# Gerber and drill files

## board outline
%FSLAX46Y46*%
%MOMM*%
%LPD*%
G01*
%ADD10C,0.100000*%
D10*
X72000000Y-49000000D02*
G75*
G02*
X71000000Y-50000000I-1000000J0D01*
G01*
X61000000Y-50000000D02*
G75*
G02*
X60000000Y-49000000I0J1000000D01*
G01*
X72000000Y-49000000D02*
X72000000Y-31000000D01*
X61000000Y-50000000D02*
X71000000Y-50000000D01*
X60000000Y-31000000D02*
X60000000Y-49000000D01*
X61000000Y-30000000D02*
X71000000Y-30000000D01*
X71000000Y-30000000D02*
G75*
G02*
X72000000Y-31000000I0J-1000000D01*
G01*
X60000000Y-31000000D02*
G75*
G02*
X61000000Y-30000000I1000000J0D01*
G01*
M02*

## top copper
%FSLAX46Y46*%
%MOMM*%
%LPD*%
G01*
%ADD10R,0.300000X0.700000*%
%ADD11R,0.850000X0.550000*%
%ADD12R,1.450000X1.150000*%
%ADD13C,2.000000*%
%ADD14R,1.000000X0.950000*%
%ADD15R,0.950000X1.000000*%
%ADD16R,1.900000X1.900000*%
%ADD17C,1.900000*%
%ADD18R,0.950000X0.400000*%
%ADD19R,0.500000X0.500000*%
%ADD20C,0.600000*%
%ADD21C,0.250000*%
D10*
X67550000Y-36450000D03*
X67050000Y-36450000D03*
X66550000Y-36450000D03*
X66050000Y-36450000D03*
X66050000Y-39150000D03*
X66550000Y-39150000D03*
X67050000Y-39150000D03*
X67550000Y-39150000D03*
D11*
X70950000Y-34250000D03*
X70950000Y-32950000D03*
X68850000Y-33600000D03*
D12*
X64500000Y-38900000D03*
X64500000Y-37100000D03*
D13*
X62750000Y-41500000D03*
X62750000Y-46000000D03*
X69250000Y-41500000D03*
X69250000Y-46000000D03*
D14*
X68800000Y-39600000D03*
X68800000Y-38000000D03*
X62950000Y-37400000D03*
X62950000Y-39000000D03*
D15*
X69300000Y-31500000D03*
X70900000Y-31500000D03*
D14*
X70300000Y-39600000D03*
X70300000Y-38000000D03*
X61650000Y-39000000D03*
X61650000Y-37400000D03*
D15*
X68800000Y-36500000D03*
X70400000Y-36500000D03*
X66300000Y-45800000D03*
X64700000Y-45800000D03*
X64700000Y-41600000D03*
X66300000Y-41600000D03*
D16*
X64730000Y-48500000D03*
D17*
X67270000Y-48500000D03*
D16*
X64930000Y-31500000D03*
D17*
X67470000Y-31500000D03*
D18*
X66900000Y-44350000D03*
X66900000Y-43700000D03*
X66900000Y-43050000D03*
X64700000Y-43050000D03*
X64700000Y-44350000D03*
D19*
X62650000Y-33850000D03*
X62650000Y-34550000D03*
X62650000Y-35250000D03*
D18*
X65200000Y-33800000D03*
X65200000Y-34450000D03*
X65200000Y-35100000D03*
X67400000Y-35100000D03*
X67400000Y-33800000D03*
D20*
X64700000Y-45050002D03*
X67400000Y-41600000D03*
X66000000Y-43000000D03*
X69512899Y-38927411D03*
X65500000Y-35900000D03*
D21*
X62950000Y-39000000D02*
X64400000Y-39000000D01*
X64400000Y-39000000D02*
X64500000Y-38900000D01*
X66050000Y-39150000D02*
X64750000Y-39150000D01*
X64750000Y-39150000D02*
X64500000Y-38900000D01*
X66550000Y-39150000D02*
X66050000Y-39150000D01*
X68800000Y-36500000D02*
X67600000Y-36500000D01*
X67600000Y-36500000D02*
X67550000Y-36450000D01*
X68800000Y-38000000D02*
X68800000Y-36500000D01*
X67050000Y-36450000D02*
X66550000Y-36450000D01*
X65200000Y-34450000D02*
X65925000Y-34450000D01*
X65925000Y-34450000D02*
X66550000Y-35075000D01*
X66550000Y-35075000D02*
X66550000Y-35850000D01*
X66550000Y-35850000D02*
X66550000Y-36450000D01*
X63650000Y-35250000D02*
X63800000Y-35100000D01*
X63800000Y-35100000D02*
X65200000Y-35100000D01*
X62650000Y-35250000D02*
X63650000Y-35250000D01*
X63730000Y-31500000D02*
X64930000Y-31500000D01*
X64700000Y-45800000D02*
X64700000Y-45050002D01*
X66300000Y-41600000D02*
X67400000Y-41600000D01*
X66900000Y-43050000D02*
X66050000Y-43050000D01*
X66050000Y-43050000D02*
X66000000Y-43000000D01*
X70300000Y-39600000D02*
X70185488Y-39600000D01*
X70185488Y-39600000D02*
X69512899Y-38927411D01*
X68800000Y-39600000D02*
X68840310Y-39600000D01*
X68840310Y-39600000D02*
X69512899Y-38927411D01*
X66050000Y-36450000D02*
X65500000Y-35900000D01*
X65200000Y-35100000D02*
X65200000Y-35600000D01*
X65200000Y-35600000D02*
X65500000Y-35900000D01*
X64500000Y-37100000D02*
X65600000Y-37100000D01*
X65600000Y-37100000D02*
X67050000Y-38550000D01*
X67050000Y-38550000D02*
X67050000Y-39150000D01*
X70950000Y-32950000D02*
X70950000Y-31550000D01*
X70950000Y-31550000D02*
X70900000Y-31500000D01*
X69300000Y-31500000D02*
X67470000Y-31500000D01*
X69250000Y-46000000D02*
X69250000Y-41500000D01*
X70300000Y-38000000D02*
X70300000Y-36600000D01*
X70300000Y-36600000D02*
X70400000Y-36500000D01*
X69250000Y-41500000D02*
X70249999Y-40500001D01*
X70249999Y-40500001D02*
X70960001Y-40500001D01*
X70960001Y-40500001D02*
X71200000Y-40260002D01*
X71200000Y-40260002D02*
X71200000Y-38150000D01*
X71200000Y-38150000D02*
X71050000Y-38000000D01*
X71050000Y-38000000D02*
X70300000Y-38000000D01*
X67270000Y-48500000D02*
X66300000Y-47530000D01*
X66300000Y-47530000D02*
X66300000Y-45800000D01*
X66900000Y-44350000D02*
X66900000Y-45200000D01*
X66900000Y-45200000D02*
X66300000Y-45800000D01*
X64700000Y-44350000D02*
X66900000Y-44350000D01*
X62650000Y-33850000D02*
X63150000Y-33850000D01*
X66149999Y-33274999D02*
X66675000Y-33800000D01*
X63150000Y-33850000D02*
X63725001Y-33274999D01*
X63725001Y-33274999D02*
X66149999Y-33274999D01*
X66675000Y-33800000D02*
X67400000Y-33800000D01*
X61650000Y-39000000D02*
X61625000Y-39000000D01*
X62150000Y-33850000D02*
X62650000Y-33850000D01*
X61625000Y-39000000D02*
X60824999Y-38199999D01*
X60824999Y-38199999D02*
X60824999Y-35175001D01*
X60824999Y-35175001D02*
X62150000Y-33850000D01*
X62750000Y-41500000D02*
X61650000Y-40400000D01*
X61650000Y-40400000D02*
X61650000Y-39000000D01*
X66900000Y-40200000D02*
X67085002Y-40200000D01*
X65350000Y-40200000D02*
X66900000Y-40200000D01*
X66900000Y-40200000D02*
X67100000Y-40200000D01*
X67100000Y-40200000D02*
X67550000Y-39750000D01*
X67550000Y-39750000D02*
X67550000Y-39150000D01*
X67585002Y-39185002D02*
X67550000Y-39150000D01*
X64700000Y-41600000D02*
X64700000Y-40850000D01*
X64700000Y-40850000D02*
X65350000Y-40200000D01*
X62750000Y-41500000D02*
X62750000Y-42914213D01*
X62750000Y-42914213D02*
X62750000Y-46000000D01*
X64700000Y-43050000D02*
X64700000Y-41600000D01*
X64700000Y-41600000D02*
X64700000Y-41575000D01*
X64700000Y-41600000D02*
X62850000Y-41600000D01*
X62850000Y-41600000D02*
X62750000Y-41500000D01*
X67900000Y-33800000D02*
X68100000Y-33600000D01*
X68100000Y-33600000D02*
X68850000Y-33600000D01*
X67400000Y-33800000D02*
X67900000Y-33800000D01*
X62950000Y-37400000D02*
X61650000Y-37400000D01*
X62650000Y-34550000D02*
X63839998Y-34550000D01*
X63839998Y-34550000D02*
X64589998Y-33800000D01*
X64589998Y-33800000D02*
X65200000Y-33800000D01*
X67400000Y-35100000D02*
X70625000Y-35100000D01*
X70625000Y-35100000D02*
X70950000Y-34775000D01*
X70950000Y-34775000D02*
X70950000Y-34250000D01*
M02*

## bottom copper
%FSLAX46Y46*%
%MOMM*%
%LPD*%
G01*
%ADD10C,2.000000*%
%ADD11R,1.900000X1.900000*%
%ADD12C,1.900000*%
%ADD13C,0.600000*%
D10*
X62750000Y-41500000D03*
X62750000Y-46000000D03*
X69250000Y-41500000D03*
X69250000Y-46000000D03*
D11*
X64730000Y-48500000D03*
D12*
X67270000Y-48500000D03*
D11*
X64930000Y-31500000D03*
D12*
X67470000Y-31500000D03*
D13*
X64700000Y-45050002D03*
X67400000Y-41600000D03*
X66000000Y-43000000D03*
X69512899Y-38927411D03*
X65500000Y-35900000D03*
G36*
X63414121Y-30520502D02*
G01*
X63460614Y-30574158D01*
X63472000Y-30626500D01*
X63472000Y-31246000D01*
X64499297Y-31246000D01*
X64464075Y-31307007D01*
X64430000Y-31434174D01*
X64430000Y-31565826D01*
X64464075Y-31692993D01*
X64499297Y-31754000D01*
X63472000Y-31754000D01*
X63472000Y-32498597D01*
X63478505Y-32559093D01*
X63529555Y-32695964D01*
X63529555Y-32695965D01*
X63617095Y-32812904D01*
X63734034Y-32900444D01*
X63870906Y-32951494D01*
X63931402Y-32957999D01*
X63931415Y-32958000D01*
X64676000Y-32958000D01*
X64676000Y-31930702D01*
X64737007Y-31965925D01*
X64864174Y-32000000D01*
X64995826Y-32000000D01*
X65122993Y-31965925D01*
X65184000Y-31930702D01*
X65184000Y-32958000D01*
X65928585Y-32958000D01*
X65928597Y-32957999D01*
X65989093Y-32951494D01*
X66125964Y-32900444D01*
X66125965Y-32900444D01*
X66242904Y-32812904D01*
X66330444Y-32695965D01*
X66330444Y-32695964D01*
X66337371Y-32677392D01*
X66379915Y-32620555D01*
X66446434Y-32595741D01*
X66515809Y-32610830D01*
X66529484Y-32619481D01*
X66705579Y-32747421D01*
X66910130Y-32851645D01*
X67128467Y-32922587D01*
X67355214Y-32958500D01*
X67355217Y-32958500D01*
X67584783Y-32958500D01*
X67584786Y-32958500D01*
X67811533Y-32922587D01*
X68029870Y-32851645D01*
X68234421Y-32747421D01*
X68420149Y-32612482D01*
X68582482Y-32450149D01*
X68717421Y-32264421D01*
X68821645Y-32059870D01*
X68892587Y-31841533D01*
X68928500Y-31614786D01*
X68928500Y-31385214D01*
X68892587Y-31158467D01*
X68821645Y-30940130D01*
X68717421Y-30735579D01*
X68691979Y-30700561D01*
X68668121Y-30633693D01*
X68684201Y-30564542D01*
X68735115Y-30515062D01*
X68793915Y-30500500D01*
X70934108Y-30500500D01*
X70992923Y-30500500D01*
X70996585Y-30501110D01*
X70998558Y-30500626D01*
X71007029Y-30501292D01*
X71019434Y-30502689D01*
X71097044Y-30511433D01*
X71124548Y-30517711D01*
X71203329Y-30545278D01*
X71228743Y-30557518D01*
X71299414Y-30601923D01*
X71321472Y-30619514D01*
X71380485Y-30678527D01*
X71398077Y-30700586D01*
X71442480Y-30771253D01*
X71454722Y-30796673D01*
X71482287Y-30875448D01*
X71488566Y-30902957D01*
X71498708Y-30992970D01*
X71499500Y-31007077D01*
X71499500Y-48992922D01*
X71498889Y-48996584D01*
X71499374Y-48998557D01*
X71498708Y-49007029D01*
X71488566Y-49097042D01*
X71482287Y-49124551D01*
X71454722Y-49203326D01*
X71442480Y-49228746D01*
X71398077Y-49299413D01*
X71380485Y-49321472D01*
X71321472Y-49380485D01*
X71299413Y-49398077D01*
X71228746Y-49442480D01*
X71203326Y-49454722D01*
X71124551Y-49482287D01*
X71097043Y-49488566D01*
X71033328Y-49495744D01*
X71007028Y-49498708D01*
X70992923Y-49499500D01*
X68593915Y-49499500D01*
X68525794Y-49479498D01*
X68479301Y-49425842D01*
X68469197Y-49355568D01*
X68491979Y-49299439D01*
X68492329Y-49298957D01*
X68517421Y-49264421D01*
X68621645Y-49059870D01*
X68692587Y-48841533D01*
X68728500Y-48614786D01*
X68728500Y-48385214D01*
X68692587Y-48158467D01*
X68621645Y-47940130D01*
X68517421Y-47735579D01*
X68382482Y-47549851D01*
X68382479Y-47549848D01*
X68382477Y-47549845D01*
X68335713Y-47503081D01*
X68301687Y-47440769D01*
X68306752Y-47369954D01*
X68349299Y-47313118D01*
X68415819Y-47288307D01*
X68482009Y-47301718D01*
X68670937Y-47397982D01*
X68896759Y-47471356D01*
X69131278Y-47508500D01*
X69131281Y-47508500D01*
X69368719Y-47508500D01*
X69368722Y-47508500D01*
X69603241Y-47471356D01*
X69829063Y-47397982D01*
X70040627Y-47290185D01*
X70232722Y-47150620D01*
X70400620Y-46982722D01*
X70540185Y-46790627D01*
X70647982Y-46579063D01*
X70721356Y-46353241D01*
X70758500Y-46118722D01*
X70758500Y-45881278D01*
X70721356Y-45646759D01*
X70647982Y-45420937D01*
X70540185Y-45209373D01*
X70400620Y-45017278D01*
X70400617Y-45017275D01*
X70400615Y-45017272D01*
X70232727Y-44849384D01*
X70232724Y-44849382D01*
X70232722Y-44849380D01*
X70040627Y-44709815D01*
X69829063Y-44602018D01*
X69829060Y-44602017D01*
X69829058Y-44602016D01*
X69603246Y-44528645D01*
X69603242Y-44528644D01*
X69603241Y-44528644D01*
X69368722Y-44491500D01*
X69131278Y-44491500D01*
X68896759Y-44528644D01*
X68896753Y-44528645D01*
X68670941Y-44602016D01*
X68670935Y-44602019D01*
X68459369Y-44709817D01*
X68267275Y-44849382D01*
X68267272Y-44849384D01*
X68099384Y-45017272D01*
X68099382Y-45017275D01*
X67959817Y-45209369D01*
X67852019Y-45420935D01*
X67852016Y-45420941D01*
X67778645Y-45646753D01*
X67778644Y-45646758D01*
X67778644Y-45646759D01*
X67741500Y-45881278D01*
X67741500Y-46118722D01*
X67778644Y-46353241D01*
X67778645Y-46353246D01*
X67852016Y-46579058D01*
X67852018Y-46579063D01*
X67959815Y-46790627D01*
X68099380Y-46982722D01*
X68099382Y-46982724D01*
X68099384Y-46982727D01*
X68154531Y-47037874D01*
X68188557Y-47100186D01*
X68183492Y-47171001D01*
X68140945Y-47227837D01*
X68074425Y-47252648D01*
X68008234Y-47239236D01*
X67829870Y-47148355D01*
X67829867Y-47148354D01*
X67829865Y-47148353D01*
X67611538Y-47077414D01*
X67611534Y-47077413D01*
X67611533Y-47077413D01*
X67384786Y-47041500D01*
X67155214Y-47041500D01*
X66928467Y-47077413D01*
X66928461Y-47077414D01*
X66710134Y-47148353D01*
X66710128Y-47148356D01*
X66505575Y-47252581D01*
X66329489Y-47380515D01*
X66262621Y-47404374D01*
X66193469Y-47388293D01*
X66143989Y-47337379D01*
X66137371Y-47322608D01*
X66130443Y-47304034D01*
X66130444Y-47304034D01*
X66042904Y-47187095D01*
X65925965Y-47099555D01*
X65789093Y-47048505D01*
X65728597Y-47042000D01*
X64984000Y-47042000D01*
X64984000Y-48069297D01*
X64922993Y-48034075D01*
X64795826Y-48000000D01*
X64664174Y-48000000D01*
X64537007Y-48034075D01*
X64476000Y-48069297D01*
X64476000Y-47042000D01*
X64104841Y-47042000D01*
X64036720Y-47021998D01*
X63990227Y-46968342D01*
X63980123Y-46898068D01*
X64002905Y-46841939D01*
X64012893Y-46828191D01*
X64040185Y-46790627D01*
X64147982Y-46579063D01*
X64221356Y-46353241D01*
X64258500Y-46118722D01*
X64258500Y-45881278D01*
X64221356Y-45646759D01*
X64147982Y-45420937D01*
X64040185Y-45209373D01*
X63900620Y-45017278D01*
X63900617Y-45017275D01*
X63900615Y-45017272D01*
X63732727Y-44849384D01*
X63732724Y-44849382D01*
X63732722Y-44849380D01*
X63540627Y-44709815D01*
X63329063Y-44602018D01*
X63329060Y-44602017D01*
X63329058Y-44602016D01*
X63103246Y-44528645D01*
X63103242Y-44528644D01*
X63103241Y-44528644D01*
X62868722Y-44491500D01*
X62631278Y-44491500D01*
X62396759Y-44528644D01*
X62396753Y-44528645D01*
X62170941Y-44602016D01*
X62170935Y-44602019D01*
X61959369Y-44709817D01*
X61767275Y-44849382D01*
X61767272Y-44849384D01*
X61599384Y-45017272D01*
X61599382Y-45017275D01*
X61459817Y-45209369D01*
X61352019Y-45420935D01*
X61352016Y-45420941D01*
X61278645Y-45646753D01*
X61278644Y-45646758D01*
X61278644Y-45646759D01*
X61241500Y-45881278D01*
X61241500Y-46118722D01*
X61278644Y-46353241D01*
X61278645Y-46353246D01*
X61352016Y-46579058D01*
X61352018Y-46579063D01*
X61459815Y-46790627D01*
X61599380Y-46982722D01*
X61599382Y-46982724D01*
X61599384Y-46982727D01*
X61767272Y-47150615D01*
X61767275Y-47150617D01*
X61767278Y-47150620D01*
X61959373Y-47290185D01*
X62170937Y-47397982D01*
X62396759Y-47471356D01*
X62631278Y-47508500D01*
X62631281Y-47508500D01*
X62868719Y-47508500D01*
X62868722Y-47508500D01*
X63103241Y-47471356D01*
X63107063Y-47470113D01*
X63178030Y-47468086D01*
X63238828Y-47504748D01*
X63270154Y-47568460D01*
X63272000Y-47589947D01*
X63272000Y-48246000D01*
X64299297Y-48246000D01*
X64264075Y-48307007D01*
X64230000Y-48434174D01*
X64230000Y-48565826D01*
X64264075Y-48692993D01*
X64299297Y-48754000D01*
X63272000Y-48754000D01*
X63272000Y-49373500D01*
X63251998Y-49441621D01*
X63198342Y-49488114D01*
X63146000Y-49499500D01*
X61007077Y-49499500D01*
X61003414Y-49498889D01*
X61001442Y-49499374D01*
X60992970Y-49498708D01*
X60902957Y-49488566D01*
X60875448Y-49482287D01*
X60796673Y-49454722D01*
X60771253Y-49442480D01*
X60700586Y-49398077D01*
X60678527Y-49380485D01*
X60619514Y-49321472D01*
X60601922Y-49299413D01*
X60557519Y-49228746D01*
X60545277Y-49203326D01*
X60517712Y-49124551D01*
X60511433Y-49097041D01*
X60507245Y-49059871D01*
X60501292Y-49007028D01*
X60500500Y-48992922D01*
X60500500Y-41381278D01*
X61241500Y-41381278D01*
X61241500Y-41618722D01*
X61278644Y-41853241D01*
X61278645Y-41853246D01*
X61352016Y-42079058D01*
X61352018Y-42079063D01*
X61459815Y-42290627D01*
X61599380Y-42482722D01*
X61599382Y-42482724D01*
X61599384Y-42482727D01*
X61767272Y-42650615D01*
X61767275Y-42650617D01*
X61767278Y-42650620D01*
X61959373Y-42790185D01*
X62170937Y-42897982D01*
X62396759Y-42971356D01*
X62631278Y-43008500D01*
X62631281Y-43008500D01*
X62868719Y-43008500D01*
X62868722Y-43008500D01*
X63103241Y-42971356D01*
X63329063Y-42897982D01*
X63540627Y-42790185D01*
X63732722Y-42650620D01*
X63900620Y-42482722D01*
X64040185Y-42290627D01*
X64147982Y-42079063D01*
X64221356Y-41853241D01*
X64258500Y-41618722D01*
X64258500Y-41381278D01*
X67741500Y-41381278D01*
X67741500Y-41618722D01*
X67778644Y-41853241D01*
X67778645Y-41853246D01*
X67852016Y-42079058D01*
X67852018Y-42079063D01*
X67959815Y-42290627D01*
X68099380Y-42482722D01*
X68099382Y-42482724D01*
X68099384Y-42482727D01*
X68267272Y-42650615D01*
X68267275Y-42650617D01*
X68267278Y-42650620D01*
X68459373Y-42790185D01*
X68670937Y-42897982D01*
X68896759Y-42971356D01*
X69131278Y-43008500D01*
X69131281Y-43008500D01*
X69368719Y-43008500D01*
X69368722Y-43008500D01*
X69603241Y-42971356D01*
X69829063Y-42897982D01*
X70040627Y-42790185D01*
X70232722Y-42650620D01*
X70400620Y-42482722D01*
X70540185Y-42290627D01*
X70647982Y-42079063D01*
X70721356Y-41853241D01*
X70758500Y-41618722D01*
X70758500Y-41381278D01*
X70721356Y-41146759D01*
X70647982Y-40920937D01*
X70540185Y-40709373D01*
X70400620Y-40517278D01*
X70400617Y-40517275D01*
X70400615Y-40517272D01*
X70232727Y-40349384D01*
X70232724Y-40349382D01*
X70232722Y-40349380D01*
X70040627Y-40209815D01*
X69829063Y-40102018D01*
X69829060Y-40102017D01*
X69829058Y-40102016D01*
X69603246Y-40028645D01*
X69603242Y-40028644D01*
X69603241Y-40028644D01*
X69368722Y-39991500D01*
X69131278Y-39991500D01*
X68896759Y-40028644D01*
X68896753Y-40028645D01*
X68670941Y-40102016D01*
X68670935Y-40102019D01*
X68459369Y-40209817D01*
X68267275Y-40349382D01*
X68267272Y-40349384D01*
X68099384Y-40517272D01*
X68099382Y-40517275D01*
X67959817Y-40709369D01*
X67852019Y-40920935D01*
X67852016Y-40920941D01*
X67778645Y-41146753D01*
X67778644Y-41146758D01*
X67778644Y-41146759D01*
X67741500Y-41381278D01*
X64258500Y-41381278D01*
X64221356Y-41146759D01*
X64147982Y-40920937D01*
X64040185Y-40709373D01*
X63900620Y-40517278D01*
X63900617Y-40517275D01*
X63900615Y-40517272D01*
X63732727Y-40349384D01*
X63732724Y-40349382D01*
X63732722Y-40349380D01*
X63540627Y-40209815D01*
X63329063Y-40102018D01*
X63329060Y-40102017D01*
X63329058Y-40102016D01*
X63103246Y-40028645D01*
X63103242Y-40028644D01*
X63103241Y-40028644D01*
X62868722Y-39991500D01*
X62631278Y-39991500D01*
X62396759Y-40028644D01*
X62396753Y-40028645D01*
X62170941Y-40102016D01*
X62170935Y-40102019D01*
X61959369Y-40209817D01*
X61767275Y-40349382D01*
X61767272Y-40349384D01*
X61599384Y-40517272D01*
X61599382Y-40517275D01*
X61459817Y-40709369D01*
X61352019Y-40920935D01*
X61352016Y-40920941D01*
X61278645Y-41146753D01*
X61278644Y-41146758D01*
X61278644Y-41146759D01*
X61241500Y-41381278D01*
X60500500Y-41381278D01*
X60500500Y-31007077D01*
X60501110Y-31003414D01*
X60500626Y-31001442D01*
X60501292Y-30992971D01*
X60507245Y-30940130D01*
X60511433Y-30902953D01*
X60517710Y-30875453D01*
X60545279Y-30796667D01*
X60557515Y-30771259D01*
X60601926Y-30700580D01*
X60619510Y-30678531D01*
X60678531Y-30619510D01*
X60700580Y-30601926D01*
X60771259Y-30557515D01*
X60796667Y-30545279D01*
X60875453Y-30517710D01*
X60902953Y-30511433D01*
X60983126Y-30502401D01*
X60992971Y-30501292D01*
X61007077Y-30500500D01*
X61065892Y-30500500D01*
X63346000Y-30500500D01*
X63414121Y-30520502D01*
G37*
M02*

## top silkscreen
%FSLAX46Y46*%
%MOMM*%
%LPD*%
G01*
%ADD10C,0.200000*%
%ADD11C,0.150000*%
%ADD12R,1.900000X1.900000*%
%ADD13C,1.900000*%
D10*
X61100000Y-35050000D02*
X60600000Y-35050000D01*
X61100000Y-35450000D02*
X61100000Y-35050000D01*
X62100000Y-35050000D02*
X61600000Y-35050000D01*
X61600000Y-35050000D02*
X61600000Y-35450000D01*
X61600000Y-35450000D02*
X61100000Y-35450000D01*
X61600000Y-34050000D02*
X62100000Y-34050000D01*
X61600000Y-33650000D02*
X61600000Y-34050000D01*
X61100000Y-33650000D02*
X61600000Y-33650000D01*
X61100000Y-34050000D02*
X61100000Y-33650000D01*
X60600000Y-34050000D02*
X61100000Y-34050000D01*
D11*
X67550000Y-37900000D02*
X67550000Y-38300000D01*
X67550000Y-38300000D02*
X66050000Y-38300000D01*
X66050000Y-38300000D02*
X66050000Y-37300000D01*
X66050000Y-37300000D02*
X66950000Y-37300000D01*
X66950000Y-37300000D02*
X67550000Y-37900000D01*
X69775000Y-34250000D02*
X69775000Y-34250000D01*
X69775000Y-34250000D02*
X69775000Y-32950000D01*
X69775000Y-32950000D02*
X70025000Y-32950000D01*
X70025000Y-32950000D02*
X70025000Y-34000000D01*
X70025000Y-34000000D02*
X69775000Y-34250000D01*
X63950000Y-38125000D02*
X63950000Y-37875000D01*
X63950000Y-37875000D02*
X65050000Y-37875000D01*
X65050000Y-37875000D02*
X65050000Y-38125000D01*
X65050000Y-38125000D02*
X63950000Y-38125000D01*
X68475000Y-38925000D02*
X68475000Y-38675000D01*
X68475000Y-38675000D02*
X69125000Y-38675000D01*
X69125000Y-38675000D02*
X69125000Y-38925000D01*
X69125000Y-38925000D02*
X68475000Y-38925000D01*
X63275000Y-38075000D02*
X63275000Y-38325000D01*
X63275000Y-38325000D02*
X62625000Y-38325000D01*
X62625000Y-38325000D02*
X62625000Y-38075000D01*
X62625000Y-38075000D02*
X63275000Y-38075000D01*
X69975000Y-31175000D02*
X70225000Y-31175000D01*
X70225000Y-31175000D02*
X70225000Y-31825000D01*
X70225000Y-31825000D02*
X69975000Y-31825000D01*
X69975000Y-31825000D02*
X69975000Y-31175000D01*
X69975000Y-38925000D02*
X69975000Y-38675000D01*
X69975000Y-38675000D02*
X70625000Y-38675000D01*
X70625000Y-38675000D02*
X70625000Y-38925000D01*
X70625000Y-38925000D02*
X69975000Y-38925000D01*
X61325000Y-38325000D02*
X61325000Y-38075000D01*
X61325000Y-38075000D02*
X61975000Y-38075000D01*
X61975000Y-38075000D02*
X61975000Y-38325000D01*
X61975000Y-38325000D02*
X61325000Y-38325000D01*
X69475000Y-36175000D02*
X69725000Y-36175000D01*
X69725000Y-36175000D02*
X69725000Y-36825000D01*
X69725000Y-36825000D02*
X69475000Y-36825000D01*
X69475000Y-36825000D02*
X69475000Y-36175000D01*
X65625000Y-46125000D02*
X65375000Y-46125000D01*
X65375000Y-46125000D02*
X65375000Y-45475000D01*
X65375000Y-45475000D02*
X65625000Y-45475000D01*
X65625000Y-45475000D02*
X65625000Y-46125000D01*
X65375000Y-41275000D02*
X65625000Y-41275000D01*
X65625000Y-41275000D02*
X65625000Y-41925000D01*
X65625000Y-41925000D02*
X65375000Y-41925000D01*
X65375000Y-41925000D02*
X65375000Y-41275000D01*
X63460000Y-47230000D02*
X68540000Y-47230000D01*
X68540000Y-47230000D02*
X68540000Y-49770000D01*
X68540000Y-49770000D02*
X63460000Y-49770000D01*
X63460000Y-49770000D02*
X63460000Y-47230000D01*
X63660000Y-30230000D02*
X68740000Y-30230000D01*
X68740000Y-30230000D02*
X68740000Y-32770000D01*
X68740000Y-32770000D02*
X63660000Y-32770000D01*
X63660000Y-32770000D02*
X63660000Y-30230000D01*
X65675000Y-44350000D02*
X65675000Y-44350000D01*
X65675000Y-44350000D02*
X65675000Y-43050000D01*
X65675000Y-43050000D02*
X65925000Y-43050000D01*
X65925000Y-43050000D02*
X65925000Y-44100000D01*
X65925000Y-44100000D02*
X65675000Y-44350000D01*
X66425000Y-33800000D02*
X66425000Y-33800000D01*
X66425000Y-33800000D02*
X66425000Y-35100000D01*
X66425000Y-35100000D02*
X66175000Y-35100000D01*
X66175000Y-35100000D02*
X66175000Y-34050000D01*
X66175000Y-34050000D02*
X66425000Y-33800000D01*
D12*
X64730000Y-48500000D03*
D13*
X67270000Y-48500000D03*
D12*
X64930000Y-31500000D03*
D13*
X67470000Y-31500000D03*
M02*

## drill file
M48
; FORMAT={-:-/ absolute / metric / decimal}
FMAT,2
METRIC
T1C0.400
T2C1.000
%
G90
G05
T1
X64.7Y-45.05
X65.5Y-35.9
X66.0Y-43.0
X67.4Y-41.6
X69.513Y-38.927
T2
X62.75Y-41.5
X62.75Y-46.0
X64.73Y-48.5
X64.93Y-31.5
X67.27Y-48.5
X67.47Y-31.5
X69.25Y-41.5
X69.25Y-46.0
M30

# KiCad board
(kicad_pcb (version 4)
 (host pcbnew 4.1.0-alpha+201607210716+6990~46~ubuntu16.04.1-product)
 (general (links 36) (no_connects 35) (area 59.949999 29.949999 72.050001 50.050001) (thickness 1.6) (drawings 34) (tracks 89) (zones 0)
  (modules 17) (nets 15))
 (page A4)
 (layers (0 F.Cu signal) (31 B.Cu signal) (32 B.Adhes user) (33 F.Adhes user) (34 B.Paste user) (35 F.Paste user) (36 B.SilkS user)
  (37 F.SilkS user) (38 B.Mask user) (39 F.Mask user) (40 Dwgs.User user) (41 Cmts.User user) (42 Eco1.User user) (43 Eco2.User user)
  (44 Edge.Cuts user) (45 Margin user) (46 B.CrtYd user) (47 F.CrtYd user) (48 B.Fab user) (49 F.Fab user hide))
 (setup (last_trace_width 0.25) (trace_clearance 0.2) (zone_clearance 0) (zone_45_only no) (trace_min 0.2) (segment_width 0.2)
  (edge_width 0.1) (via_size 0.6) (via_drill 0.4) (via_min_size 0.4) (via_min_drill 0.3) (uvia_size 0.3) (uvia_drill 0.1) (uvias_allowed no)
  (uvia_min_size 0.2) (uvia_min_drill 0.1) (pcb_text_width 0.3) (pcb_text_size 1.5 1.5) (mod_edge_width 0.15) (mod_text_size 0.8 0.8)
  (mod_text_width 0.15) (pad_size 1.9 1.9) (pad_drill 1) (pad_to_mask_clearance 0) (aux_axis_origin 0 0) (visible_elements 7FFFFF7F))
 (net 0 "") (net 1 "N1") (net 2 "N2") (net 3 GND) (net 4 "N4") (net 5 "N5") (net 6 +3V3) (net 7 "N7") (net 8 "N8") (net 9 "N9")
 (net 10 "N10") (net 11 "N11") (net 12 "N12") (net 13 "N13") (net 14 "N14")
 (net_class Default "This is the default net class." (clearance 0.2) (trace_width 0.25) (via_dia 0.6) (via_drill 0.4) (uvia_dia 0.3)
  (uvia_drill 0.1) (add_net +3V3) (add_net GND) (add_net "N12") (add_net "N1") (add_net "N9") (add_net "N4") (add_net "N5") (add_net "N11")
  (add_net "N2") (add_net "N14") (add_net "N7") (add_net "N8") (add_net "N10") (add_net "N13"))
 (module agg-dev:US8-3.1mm (layer F.Cu) (at 66.8 37.8 270)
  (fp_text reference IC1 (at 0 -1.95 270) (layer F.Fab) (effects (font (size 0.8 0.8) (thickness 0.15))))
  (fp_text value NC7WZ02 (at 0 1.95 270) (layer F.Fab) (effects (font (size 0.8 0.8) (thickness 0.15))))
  (fp_line (start 0.1 -0.75) (end 0.5 -0.75) (layer F.SilkS) (width 0.15))
  (fp_line (start 0.5 -0.75) (end 0.5 0.75) (layer F.SilkS) (width 0.15))
  (fp_line (start 0.5 0.75) (end -0.5 0.75) (layer F.SilkS) (width 0.15))
  (fp_line (start -0.5 0.75) (end -0.5 -0.15) (layer F.SilkS) (width 0.15))
  (fp_line (start -0.5 -0.15) (end 0.1 -0.75) (layer F.SilkS) (width 0.15))
  (pad 1 smd rect (at -1.35 -0.75 270) (size 0.7 0.3) (layers F.Cu F.Paste F.Mask) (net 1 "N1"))
  (pad 2 smd rect (at -1.35 -0.25 270) (size 0.7 0.3) (layers F.Cu F.Paste F.Mask) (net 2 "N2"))
  (pad 3 smd rect (at -1.35 0.25 270) (size 0.7 0.3) (layers F.Cu F.Paste F.Mask) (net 2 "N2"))
  (pad 4 smd rect (at -1.35 0.75 270) (size 0.7 0.3) (layers F.Cu F.Paste F.Mask) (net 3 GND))
  (pad 5 smd rect (at 1.35 0.75 270) (size 0.7 0.3) (layers F.Cu F.Paste F.Mask) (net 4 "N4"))
  (pad 6 smd rect (at 1.35 0.25 270) (size 0.7 0.3) (layers F.Cu F.Paste F.Mask) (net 4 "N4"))
  (pad 7 smd rect (at 1.35 -0.25 270) (size 0.7 0.3) (layers F.Cu F.Paste F.Mask) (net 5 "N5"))
  (pad 8 smd rect (at 1.35 -0.75 270) (size 0.7 0.3) (layers F.Cu F.Paste F.Mask) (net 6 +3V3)))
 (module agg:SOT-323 (layer F.Cu) (at 69.9 33.6 180)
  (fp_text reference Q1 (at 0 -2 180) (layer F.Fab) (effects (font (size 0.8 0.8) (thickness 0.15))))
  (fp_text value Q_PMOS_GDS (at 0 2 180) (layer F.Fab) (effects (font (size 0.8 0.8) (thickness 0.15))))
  (fp_line (start 0.125 -0.65) (end 0.125 -0.65) (layer F.SilkS) (width 0.15))
  (fp_line (start 0.125 -0.65) (end 0.125 0.65) (layer F.SilkS) (width 0.15))
  (fp_line (start 0.125 0.65) (end -0.125 0.65) (layer F.SilkS) (width 0.15))
  (fp_line (start -0.125 0.65) (end -0.125 -0.4) (layer F.SilkS) (width 0.15))
  (fp_line (start -0.125 -0.4) (end 0.125 -0.65) (layer F.SilkS) (width 0.15))
  (pad 1 smd rect (at -1.05 -0.65 180) (size 0.85 0.55) (layers F.Cu F.Paste F.Mask) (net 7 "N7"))
  (pad 2 smd rect (at -1.05 0.65 180) (size 0.85 0.55) (layers F.Cu F.Paste F.Mask) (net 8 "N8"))
  (pad 3 smd rect (at 1.05 0 180) (size 0.85 0.55) (layers F.Cu F.Paste F.Mask) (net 6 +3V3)))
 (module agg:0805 (layer F.Cu) (at 64.5 38 90)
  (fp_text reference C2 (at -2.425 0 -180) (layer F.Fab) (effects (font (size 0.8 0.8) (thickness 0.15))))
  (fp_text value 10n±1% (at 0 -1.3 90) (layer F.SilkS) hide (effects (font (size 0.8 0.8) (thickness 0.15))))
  (fp_line (start -0.125 -0.55) (end 0.125 -0.55) (layer F.SilkS) (width 0.15))
  (fp_line (start 0.125 -0.55) (end 0.125 0.55) (layer F.SilkS) (width 0.15))
  (fp_line (start 0.125 0.55) (end -0.125 0.55) (layer F.SilkS) (width 0.15))
  (fp_line (start -0.125 0.55) (end -0.125 -0.55) (layer F.SilkS) (width 0.15))
  (pad 1 smd rect (at -0.9 0 90) (size 1.15 1.45) (layers F.Cu F.Paste F.Mask) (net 4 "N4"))
  (pad 2 smd rect (at 0.9 0 90) (size 1.15 1.45) (layers F.Cu F.Paste F.Mask) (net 5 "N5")))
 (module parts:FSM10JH (layer B.Cu) (at 62.75 41.5 180)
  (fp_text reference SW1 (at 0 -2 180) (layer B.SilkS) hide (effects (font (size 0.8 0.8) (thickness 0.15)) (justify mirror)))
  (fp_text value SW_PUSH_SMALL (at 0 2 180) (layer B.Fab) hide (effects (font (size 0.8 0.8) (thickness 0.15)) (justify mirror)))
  (pad 1 thru_hole circle (at 0 0 180) (size 2 2) (drill 1) (layers *.Cu *.Mask B.SilkS) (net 6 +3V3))
  (pad 1 thru_hole circle (at 0 -4.5 180) (size 2 2) (drill 1) (layers *.Cu *.Mask B.SilkS) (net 6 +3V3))
  (pad 2 thru_hole circle (at -6.5 0 180) (size 2 2) (drill 1) (layers *.Cu *.Mask B.SilkS) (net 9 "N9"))
  (pad 2 thru_hole circle (at -6.5 -4.5 180) (size 2 2) (drill 1) (layers *.Cu *.Mask B.SilkS) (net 9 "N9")))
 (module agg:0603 (layer F.Cu) (at 68.8 38.8 90)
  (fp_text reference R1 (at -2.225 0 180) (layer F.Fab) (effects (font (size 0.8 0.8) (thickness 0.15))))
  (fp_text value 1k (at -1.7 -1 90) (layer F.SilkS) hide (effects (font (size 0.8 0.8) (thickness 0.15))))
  (fp_line (start -0.125 -0.325) (end 0.125 -0.325) (layer F.SilkS) (width 0.15))
  (fp_line (start 0.125 -0.325) (end 0.125 0.325) (layer F.SilkS) (width 0.15))
  (fp_line (start 0.125 0.325) (end -0.125 0.325) (layer F.SilkS) (width 0.15))
  (fp_line (start -0.125 0.325) (end -0.125 -0.325) (layer F.SilkS) (width 0.15))
  (pad 1 smd rect (at -0.8 0 90) (size 0.95 1) (layers F.Cu F.Paste F.Mask) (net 3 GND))
  (pad 2 smd rect (at 0.8 0 90) (size 0.95 1) (layers F.Cu F.Paste F.Mask) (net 1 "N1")))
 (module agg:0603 (layer F.Cu) (at 62.95 38.2 270)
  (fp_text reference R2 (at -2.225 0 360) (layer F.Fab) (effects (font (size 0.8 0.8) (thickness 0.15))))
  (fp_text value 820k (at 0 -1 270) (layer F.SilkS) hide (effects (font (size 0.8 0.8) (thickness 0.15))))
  (fp_line (start -0.125 -0.325) (end 0.125 -0.325) (layer F.SilkS) (width 0.15))
  (fp_line (start 0.125 -0.325) (end 0.125 0.325) (layer F.SilkS) (width 0.15))
  (fp_line (start 0.125 0.325) (end -0.125 0.325) (layer F.SilkS) (width 0.15))
  (fp_line (start -0.125 0.325) (end -0.125 -0.325) (layer F.SilkS) (width 0.15))
  (pad 1 smd rect (at -0.8 0 270) (size 0.95 1) (layers F.Cu F.Paste F.Mask) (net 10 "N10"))
  (pad 2 smd rect (at 0.8 0 270) (size 0.95 1) (layers F.Cu F.Paste F.Mask) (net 4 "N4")))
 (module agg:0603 (layer F.Cu) (at 70.1 31.5)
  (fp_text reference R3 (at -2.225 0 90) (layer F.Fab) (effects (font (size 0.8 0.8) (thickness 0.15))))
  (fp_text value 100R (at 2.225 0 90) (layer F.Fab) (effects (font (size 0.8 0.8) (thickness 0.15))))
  (fp_line (start -0.125 -0.325) (end 0.125 -0.325) (layer F.SilkS) (width 0.15))
  (fp_line (start 0.125 -0.325) (end 0.125 0.325) (layer F.SilkS) (width 0.15))
  (fp_line (start 0.125 0.325) (end -0.125 0.325) (layer F.SilkS) (width 0.15))
  (fp_line (start -0.125 0.325) (end -0.125 -0.325) (layer F.SilkS) (width 0.15))
  (pad 1 smd rect (at -0.8 0) (size 0.95 1) (layers F.Cu F.Paste F.Mask) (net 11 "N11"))
  (pad 2 smd rect (at 0.8 0) (size 0.95 1) (layers F.Cu F.Paste F.Mask) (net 8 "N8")))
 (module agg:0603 (layer F.Cu) (at 70.3 38.8 90)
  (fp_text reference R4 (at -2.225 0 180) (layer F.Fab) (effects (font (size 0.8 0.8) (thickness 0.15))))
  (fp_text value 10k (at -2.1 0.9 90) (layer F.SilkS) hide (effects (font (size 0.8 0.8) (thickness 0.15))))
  (fp_line (start -0.125 -0.325) (end 0.125 -0.325) (layer F.SilkS) (width 0.15))
  (fp_line (start 0.125 -0.325) (end 0.125 0.325) (layer F.SilkS) (width 0.15))
  (fp_line (start 0.125 0.325) (end -0.125 0.325) (layer F.SilkS) (width 0.15))
  (fp_line (start -0.125 0.325) (end -0.125 -0.325) (layer F.SilkS) (width 0.15))
  (pad 1 smd rect (at -0.8 0 90) (size 0.95 1) (layers F.Cu F.Paste F.Mask) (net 3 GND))
  (pad 2 smd rect (at 0.8 0 90) (size 0.95 1) (layers F.Cu F.Paste F.Mask) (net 9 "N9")))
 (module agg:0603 (layer F.Cu) (at 61.65 38.2 90)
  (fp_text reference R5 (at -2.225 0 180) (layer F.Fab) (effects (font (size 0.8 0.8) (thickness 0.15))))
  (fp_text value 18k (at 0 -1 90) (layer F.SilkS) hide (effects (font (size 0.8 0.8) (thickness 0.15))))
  (fp_line (start -0.125 -0.325) (end 0.125 -0.325) (layer F.SilkS) (width 0.15))
  (fp_line (start 0.125 -0.325) (end 0.125 0.325) (layer F.SilkS) (width 0.15))
  (fp_line (start 0.125 0.325) (end -0.125 0.325) (layer F.SilkS) (width 0.15))
  (fp_line (start -0.125 0.325) (end -0.125 -0.325) (layer F.SilkS) (width 0.15))
  (pad 1 smd rect (at -0.8 0 90) (size 0.95 1) (layers F.Cu F.Paste F.Mask) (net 6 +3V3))
  (pad 2 smd rect (at 0.8 0 90) (size 0.95 1) (layers F.Cu F.Paste F.Mask) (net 10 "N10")))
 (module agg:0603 (layer F.Cu) (at 69.6 36.5)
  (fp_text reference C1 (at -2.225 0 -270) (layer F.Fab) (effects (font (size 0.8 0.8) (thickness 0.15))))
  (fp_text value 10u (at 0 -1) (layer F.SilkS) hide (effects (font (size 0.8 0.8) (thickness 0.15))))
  (fp_line (start -0.125 -0.325) (end 0.125 -0.325) (layer F.SilkS) (width 0.15))
  (fp_line (start 0.125 -0.325) (end 0.125 0.325) (layer F.SilkS) (width 0.15))
  (fp_line (start 0.125 0.325) (end -0.125 0.325) (layer F.SilkS) (width 0.15))
  (fp_line (start -0.125 0.325) (end -0.125 -0.325) (layer F.SilkS) (width 0.15))
  (pad 1 smd rect (at -0.8 0) (size 0.95 1) (layers F.Cu F.Paste F.Mask) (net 1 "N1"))
  (pad 2 smd rect (at 0.8 0) (size 0.95 1) (layers F.Cu F.Paste F.Mask) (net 9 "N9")))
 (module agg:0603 (layer F.Cu) (at 65.5 45.8 180)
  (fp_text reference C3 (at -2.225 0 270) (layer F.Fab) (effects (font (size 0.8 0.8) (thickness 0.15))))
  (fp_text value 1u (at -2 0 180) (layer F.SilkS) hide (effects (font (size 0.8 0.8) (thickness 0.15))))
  (fp_line (start -0.125 -0.325) (end 0.125 -0.325) (layer F.SilkS) (width 0.15))
  (fp_line (start 0.125 -0.325) (end 0.125 0.325) (layer F.SilkS) (width 0.15))
  (fp_line (start 0.125 0.325) (end -0.125 0.325) (layer F.SilkS) (width 0.15))
  (fp_line (start -0.125 0.325) (end -0.125 -0.325) (layer F.SilkS) (width 0.15))
  (pad 1 smd rect (at -0.8 0 180) (size 0.95 1) (layers F.Cu F.Paste F.Mask) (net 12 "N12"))
  (pad 2 smd rect (at 0.8 0 180) (size 0.95 1) (layers F.Cu F.Paste F.Mask) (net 3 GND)))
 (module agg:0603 (layer F.Cu) (at 65.5 41.6)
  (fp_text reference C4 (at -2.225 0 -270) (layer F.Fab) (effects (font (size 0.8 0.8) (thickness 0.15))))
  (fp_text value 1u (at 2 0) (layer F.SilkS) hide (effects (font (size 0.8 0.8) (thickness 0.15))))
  (fp_line (start -0.125 -0.325) (end 0.125 -0.325) (layer F.SilkS) (width 0.15))
  (fp_line (start 0.125 -0.325) (end 0.125 0.325) (layer F.SilkS) (width 0.15))
  (fp_line (start 0.125 0.325) (end -0.125 0.325) (layer F.SilkS) (width 0.15))
  (fp_line (start -0.125 0.325) (end -0.125 -0.325) (layer F.SilkS) (width 0.15))
  (pad 1 smd rect (at -0.8 0) (size 0.95 1) (layers F.Cu F.Paste F.Mask) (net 6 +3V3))
  (pad 2 smd rect (at 0.8 0) (size 0.95 1) (layers F.Cu F.Paste F.Mask) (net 3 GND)))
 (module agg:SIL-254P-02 (layer F.Cu) (at 66 48.5)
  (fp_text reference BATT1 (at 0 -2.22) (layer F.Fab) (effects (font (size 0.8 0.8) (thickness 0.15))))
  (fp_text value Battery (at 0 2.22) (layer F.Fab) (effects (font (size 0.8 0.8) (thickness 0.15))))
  (fp_line (start -2.54 -1.27) (end 2.54 -1.27) (layer F.SilkS) (width 0.15))
  (fp_line (start 2.54 -1.27) (end 2.54 1.27) (layer F.SilkS) (width 0.15))
  (fp_line (start 2.54 1.27) (end -2.54 1.27) (layer F.SilkS) (width 0.15))
  (fp_line (start -2.54 1.27) (end -2.54 -1.27) (layer F.SilkS) (width 0.15))
  (pad 2 thru_hole rect (at -1.27 0) (size 1.9 1.9) (drill 1) (layers *.Cu *.Mask F.SilkS) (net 3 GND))
  (pad 1 thru_hole circle (at 1.27 0) (size 1.9 1.9) (drill 1) (layers *.Cu *.Mask F.SilkS) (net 12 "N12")))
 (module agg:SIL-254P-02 (layer F.Cu) (at 66.2 31.5)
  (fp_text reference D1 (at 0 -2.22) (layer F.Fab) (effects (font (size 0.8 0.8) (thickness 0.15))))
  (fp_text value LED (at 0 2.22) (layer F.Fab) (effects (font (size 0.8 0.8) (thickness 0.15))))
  (fp_line (start -2.54 -1.27) (end 2.54 -1.27) (layer F.SilkS) (width 0.15))
  (fp_line (start 2.54 -1.27) (end 2.54 1.27) (layer F.SilkS) (width 0.15))
  (fp_line (start 2.54 1.27) (end -2.54 1.27) (layer F.SilkS) (width 0.15))
  (fp_line (start -2.54 1.27) (end -2.54 -1.27) (layer F.SilkS) (width 0.15))
  (pad 1 thru_hole rect (at -1.27 0) (size 1.9 1.9) (drill 1) (layers *.Cu *.Mask F.SilkS) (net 3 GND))
  (pad 2 thru_hole circle (at 1.27 0) (size 1.9 1.9) (drill 1) (layers *.Cu *.Mask F.SilkS) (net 11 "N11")))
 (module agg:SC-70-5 (layer F.Cu) (at 65.8 43.7 180)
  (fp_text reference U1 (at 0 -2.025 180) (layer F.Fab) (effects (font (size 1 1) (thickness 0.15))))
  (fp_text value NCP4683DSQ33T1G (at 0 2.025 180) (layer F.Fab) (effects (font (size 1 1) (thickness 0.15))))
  (fp_line (start 0.125 -0.65) (end 0.125 -0.65) (layer F.SilkS) (width 0.15))
  (fp_line (start 0.125 -0.65) (end 0.125 0.65) (layer F.SilkS) (width 0.15))
  (fp_line (start 0.125 0.65) (end -0.125 0.65) (layer F.SilkS) (width 0.15))
  (fp_line (start -0.125 0.65) (end -0.125 -0.4) (layer F.SilkS) (width 0.15))
  (fp_line (start -0.125 -0.4) (end 0.125 -0.65) (layer F.SilkS) (width 0.15))
  (pad 1 smd rect (at -1.1 -0.65 180) (size 0.95 0.4) (layers F.Cu F.Paste F.Mask) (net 12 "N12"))
  (pad 2 smd rect (at -1.1 0 180) (size 0.95 0.4) (layers F.Cu F.Paste F.Mask) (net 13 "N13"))
  (pad 3 smd rect (at -1.1 0.65 180) (size 0.95 0.4) (layers F.Cu F.Paste F.Mask) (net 3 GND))
  (pad 4 smd rect (at 1.1 0.65 180) (size 0.95 0.4) (layers F.Cu F.Paste F.Mask) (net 6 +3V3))
  (pad 5 smd rect (at 1.1 -0.65 180) (size 0.95 0.4) (layers F.Cu F.Paste F.Mask) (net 12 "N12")))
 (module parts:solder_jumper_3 (layer F.Cu) (at 62.65 33.85)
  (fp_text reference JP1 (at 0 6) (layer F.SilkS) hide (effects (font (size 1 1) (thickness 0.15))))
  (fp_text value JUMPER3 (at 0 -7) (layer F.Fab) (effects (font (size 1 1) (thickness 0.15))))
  (pad 1 smd rect (at 0 0) (size 0.5 0.5) (layers F.Cu F.Mask) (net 6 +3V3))
  (pad 2 smd rect (at 0 0.7) (size 0.5 0.5) (layers F.Cu F.Mask) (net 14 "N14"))
  (pad 3 smd rect (at 0 1.4) (size 0.5 0.5) (layers F.Cu F.Mask) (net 3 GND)))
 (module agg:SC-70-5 (layer F.Cu) (at 66.3 34.45)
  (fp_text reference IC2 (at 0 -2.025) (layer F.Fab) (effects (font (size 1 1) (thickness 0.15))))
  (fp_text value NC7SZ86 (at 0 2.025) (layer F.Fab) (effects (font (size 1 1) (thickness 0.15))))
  (fp_line (start 0.125 -0.65) (end 0.125 -0.65) (layer F.SilkS) (width 0.15))
  (fp_line (start 0.125 -0.65) (end 0.125 0.65) (layer F.SilkS) (width 0.15))
  (fp_line (start 0.125 0.65) (end -0.125 0.65) (layer F.SilkS) (width 0.15))
  (fp_line (start -0.125 0.65) (end -0.125 -0.4) (layer F.SilkS) (width 0.15))
  (fp_line (start -0.125 -0.4) (end 0.125 -0.65) (layer F.SilkS) (width 0.15))
  (pad 1 smd rect (at -1.1 -0.65) (size 0.95 0.4) (layers F.Cu F.Paste F.Mask) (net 14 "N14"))
  (pad 2 smd rect (at -1.1 0) (size 0.95 0.4) (layers F.Cu F.Paste F.Mask) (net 2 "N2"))
  (pad 3 smd rect (at -1.1 0.65) (size 0.95 0.4) (layers F.Cu F.Paste F.Mask) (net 3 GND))
  (pad 4 smd rect (at 1.1 0.65) (size 0.95 0.4) (layers F.Cu F.Paste F.Mask) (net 7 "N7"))
  (pad 5 smd rect (at 1.1 -0.65) (size 0.95 0.4) (layers F.Cu F.Paste F.Mask) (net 6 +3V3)))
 (gr_line (start 61.1 35.05) (end 60.6 35.05) (layer F.SilkS) (width 0.2))
 (gr_line (start 61.1 35.45) (end 61.1 35.05) (layer F.SilkS) (width 0.2))
 (gr_line (start 62.1 35.05) (end 61.6 35.05) (layer F.SilkS) (width 0.2))
 (gr_line (start 61.6 35.05) (end 61.6 35.45) (layer F.SilkS) (width 0.2))
 (gr_line (start 61.6 35.45) (end 61.1 35.45) (layer F.SilkS) (width 0.2))
 (gr_line (start 61.6 34.05) (end 62.1 34.05) (layer F.SilkS) (width 0.2))
 (gr_line (start 61.6 33.65) (end 61.6 34.05) (layer F.SilkS) (width 0.2))
 (gr_line (start 61.1 33.65) (end 61.6 33.65) (layer F.SilkS) (width 0.2))
 (gr_line (start 61.1 34.05) (end 61.1 33.65) (layer F.SilkS) (width 0.2))
 (gr_line (start 60.6 34.05) (end 61.1 34.05) (layer F.SilkS) (width 0.2))
 (gr_arc (start 71 49) (end 72 49) (angle 90) (layer Edge.Cuts) (width 0.1))
 (gr_arc (start 61 49) (end 61 50) (angle 90) (layer Edge.Cuts) (width 0.1))
 (gr_line (start 72 49) (end 72 31) (layer Edge.Cuts) (width 0.1))
 (gr_line (start 61 50) (end 71 50) (layer Edge.Cuts) (width 0.1))
 (gr_line (start 60 31) (end 60 49) (layer Edge.Cuts) (width 0.1))
 (gr_line (start 61 30) (end 71 30) (layer Edge.Cuts) (width 0.1))
 (gr_arc (start 71 31) (end 71 30) (angle 90) (layer Edge.Cuts) (width 0.1))
 (gr_arc (start 61 31) (end 60 31) (angle 90) (layer Edge.Cuts) (width 0.1))
 (segment (start 62.95 39) (end 64.4 39) (width 0.25) (layer F.Cu) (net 4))
 (segment (start 64.4 39) (end 64.5 38.9) (width 0.25) (layer F.Cu) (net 4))
 (segment (start 66.05 39.15) (end 64.75 39.15) (width 0.25) (layer F.Cu) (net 4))
 (segment (start 64.75 39.15) (end 64.5 38.9) (width 0.25) (layer F.Cu) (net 4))
 (segment (start 66.55 39.15) (end 66.05 39.15) (width 0.25) (layer F.Cu) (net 4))
 (segment (start 68.8 36.5) (end 67.6 36.5) (width 0.25) (layer F.Cu) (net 1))
 (segment (start 67.6 36.5) (end 67.55 36.45) (width 0.25) (layer F.Cu) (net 1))
 (segment (start 68.8 38) (end 68.8 36.5) (width 0.25) (layer F.Cu) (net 1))
 (segment (start 67.05 36.45) (end 66.55 36.45) (width 0.25) (layer F.Cu) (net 2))
 (segment (start 65.2 34.45) (end 65.925 34.45) (width 0.25) (layer F.Cu) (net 2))
 (segment (start 65.925 34.45) (end 66.55 35.075) (width 0.25) (layer F.Cu) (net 2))
 (segment (start 66.55 35.075) (end 66.55 35.85) (width 0.25) (layer F.Cu) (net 2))
 (segment (start 66.55 35.85) (end 66.55 36.45) (width 0.25) (layer F.Cu) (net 2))
 (segment (start 63.65 35.25) (end 63.8 35.1) (width 0.25) (layer F.Cu) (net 3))
 (segment (start 63.8 35.1) (end 65.2 35.1) (width 0.25) (layer F.Cu) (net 3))
 (segment (start 62.65 35.25) (end 63.65 35.25) (width 0.25) (layer F.Cu) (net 3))
 (segment (start 63.73 31.5) (end 64.93 31.5) (width 0.25) (layer F.Cu) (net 3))
 (segment (start 64.7 45.8) (end 64.7 45.050002) (width 0.25) (layer F.Cu) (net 3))
 (via (at 64.7 45.050002) (size 0.6) (drill 0.4) (layers F.Cu B.Cu) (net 3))
 (segment (start 66.3 41.6) (end 67.4 41.6) (width 0.25) (layer F.Cu) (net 3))
 (via (at 67.4 41.6) (size 0.6) (drill 0.4) (layers F.Cu B.Cu) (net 3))
 (segment (start 66.9 43.05) (end 66.05 43.05) (width 0.25) (layer F.Cu) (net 3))
 (segment (start 66.05 43.05) (end 66 43) (width 0.25) (layer F.Cu) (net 3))
 (via (at 66 43) (size 0.6) (drill 0.4) (layers F.Cu B.Cu) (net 3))
 (segment (start 70.3 39.6) (end 70.185488 39.6) (width 0.25) (layer F.Cu) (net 3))
 (segment (start 70.185488 39.6) (end 69.512899 38.927411) (width 0.25) (layer F.Cu) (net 3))
 (segment (start 68.8 39.6) (end 68.84031 39.6) (width 0.25) (layer F.Cu) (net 3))
 (segment (start 68.84031 39.6) (end 69.512899 38.927411) (width 0.25) (layer F.Cu) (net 3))
 (via (at 69.512899 38.927411) (size 0.6) (drill 0.4) (layers F.Cu B.Cu) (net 3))
 (segment (start 66.05 36.45) (end 65.5 35.9) (width 0.25) (layer F.Cu) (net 3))
 (segment (start 65.2 35.1) (end 65.2 35.6) (width 0.25) (layer F.Cu) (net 3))
 (via (at 65.5 35.9) (size 0.6) (drill 0.4) (layers F.Cu B.Cu) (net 3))
 (segment (start 65.2 35.6) (end 65.5 35.9) (width 0.25) (layer F.Cu) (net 3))
 (segment (start 64.5 37.1) (end 65.6 37.1) (width 0.25) (layer F.Cu) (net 5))
 (segment (start 65.6 37.1) (end 67.05 38.55) (width 0.25) (layer F.Cu) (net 5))
 (segment (start 67.05 38.55) (end 67.05 39.15) (width 0.25) (layer F.Cu) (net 5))
 (segment (start 70.95 32.95) (end 70.95 31.55) (width 0.25) (layer F.Cu) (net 8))
 (segment (start 70.95 31.55) (end 70.9 31.5) (width 0.25) (layer F.Cu) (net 8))
 (segment (start 69.3 31.5) (end 67.47 31.5) (width 0.25) (layer F.Cu) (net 11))
 (segment (start 69.25 46) (end 69.25 41.5) (width 0.25) (layer F.Cu) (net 9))
 (segment (start 70.3 38) (end 70.3 36.6) (width 0.25) (layer F.Cu) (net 9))
 (segment (start 70.3 36.6) (end 70.4 36.5) (width 0.25) (layer F.Cu) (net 9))
 (segment (start 69.25 41.5) (end 70.249999 40.500001) (width 0.25) (layer F.Cu) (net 9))
 (segment (start 70.249999 40.500001) (end 70.960001 40.500001) (width 0.25) (layer F.Cu) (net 9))
 (segment (start 70.960001 40.500001) (end 71.2 40.260002) (width 0.25) (layer F.Cu) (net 9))
 (segment (start 71.2 40.260002) (end 71.2 38.15) (width 0.25) (layer F.Cu) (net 9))
 (segment (start 71.2 38.15) (end 71.05 38) (width 0.25) (layer F.Cu) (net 9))
 (segment (start 71.05 38) (end 70.3 38) (width 0.25) (layer F.Cu) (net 9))
 (segment (start 67.27 48.5) (end 66.3 47.53) (width 0.25) (layer F.Cu) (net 12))
 (segment (start 66.3 47.53) (end 66.3 45.8) (width 0.25) (layer F.Cu) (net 12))
 (segment (start 66.9 44.35) (end 66.9 45.2) (width 0.25) (layer F.Cu) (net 12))
 (segment (start 66.9 45.2) (end 66.3 45.8) (width 0.25) (layer F.Cu) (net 12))
 (segment (start 64.7 44.35) (end 66.9 44.35) (width 0.25) (layer F.Cu) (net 12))
 (segment (start 62.65 33.85) (end 63.15 33.85) (width 0.25) (layer F.Cu) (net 6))
 (segment (start 66.149999 33.274999) (end 66.675 33.8) (width 0.25) (layer F.Cu) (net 6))
 (segment (start 63.15 33.85) (end 63.725001 33.274999) (width 0.25) (layer F.Cu) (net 6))
 (segment (start 63.725001 33.274999) (end 66.149999 33.274999) (width 0.25) (layer F.Cu) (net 6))
 (segment (start 66.675 33.8) (end 67.4 33.8) (width 0.25) (layer F.Cu) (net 6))
 (segment (start 61.65 39) (end 61.625 39) (width 0.25) (layer F.Cu) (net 6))
 (segment (start 62.15 33.85) (end 62.65 33.85) (width 0.25) (layer F.Cu) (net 6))
 (segment (start 61.625 39) (end 60.824999 38.199999) (width 0.25) (layer F.Cu) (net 6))
 (segment (start 60.824999 38.199999) (end 60.824999 35.175001) (width 0.25) (layer F.Cu) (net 6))
 (segment (start 60.824999 35.175001) (end 62.15 33.85) (width 0.25) (layer F.Cu) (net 6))
 (segment (start 62.75 41.5) (end 61.65 40.4) (width 0.25) (layer F.Cu) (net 6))
 (segment (start 61.65 40.4) (end 61.65 39) (width 0.25) (layer F.Cu) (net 6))
 (segment (start 66.9 40.2) (end 67.085002 40.2) (width 0.25) (layer F.Cu) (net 6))
 (segment (start 65.35 40.2) (end 66.9 40.2) (width 0.25) (layer F.Cu) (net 6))
 (segment (start 66.9 40.2) (end 67.1 40.2) (width 0.25) (layer F.Cu) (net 6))
 (segment (start 67.1 40.2) (end 67.55 39.75) (width 0.25) (layer F.Cu) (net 6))
 (segment (start 67.55 39.75) (end 67.55 39.15) (width 0.25) (layer F.Cu) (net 6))
 (segment (start 67.585002 39.185002) (end 67.55 39.15) (width 0.25) (layer F.Cu) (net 6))
 (segment (start 64.7 41.6) (end 64.7 40.85) (width 0.25) (layer F.Cu) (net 6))
 (segment (start 64.7 40.85) (end 65.35 40.2) (width 0.25) (layer F.Cu) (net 6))
 (segment (start 62.75 41.5) (end 62.75 42.914213) (width 0.25) (layer F.Cu) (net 6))
 (segment (start 62.75 42.914213) (end 62.75 46) (width 0.25) (layer F.Cu) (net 6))
 (segment (start 64.7 43.05) (end 64.7 41.6) (width 0.25) (layer F.Cu) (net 6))
 (segment (start 64.7 41.6) (end 64.7 41.575) (width 0.25) (layer F.Cu) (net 6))
 (segment (start 64.7 41.6) (end 62.85 41.6) (width 0.25) (layer F.Cu) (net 6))
 (segment (start 62.85 41.6) (end 62.75 41.5) (width 0.25) (layer F.Cu) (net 6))
 (segment (start 67.9 33.8) (end 68.1 33.6) (width 0.25) (layer F.Cu) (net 6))
 (segment (start 68.1 33.6) (end 68.85 33.6) (width 0.25) (layer F.Cu) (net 6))
 (segment (start 67.4 33.8) (end 67.9 33.8) (width 0.25) (layer F.Cu) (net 6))
 (segment (start 62.95 37.4) (end 61.65 37.4) (width 0.25) (layer F.Cu) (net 10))
 (segment (start 62.65 34.55) (end 63.839998 34.55) (width 0.25) (layer F.Cu) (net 14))
 (segment (start 63.839998 34.55) (end 64.589998 33.8) (width 0.25) (layer F.Cu) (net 14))
 (segment (start 64.589998 33.8) (end 65.2 33.8) (width 0.25) (layer F.Cu) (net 14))
 (segment (start 67.4 35.1) (end 70.625 35.1) (width 0.25) (layer F.Cu) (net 7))
 (segment (start 70.625 35.1) (end 70.95 34.775) (width 0.25) (layer F.Cu) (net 7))
 (segment (start 70.95 34.775) (end 70.95 34.25) (width 0.25) (layer F.Cu) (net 7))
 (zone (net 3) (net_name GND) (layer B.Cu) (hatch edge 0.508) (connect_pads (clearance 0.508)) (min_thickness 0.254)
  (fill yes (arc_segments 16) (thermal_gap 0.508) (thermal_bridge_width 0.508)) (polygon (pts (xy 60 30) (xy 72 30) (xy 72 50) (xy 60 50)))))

